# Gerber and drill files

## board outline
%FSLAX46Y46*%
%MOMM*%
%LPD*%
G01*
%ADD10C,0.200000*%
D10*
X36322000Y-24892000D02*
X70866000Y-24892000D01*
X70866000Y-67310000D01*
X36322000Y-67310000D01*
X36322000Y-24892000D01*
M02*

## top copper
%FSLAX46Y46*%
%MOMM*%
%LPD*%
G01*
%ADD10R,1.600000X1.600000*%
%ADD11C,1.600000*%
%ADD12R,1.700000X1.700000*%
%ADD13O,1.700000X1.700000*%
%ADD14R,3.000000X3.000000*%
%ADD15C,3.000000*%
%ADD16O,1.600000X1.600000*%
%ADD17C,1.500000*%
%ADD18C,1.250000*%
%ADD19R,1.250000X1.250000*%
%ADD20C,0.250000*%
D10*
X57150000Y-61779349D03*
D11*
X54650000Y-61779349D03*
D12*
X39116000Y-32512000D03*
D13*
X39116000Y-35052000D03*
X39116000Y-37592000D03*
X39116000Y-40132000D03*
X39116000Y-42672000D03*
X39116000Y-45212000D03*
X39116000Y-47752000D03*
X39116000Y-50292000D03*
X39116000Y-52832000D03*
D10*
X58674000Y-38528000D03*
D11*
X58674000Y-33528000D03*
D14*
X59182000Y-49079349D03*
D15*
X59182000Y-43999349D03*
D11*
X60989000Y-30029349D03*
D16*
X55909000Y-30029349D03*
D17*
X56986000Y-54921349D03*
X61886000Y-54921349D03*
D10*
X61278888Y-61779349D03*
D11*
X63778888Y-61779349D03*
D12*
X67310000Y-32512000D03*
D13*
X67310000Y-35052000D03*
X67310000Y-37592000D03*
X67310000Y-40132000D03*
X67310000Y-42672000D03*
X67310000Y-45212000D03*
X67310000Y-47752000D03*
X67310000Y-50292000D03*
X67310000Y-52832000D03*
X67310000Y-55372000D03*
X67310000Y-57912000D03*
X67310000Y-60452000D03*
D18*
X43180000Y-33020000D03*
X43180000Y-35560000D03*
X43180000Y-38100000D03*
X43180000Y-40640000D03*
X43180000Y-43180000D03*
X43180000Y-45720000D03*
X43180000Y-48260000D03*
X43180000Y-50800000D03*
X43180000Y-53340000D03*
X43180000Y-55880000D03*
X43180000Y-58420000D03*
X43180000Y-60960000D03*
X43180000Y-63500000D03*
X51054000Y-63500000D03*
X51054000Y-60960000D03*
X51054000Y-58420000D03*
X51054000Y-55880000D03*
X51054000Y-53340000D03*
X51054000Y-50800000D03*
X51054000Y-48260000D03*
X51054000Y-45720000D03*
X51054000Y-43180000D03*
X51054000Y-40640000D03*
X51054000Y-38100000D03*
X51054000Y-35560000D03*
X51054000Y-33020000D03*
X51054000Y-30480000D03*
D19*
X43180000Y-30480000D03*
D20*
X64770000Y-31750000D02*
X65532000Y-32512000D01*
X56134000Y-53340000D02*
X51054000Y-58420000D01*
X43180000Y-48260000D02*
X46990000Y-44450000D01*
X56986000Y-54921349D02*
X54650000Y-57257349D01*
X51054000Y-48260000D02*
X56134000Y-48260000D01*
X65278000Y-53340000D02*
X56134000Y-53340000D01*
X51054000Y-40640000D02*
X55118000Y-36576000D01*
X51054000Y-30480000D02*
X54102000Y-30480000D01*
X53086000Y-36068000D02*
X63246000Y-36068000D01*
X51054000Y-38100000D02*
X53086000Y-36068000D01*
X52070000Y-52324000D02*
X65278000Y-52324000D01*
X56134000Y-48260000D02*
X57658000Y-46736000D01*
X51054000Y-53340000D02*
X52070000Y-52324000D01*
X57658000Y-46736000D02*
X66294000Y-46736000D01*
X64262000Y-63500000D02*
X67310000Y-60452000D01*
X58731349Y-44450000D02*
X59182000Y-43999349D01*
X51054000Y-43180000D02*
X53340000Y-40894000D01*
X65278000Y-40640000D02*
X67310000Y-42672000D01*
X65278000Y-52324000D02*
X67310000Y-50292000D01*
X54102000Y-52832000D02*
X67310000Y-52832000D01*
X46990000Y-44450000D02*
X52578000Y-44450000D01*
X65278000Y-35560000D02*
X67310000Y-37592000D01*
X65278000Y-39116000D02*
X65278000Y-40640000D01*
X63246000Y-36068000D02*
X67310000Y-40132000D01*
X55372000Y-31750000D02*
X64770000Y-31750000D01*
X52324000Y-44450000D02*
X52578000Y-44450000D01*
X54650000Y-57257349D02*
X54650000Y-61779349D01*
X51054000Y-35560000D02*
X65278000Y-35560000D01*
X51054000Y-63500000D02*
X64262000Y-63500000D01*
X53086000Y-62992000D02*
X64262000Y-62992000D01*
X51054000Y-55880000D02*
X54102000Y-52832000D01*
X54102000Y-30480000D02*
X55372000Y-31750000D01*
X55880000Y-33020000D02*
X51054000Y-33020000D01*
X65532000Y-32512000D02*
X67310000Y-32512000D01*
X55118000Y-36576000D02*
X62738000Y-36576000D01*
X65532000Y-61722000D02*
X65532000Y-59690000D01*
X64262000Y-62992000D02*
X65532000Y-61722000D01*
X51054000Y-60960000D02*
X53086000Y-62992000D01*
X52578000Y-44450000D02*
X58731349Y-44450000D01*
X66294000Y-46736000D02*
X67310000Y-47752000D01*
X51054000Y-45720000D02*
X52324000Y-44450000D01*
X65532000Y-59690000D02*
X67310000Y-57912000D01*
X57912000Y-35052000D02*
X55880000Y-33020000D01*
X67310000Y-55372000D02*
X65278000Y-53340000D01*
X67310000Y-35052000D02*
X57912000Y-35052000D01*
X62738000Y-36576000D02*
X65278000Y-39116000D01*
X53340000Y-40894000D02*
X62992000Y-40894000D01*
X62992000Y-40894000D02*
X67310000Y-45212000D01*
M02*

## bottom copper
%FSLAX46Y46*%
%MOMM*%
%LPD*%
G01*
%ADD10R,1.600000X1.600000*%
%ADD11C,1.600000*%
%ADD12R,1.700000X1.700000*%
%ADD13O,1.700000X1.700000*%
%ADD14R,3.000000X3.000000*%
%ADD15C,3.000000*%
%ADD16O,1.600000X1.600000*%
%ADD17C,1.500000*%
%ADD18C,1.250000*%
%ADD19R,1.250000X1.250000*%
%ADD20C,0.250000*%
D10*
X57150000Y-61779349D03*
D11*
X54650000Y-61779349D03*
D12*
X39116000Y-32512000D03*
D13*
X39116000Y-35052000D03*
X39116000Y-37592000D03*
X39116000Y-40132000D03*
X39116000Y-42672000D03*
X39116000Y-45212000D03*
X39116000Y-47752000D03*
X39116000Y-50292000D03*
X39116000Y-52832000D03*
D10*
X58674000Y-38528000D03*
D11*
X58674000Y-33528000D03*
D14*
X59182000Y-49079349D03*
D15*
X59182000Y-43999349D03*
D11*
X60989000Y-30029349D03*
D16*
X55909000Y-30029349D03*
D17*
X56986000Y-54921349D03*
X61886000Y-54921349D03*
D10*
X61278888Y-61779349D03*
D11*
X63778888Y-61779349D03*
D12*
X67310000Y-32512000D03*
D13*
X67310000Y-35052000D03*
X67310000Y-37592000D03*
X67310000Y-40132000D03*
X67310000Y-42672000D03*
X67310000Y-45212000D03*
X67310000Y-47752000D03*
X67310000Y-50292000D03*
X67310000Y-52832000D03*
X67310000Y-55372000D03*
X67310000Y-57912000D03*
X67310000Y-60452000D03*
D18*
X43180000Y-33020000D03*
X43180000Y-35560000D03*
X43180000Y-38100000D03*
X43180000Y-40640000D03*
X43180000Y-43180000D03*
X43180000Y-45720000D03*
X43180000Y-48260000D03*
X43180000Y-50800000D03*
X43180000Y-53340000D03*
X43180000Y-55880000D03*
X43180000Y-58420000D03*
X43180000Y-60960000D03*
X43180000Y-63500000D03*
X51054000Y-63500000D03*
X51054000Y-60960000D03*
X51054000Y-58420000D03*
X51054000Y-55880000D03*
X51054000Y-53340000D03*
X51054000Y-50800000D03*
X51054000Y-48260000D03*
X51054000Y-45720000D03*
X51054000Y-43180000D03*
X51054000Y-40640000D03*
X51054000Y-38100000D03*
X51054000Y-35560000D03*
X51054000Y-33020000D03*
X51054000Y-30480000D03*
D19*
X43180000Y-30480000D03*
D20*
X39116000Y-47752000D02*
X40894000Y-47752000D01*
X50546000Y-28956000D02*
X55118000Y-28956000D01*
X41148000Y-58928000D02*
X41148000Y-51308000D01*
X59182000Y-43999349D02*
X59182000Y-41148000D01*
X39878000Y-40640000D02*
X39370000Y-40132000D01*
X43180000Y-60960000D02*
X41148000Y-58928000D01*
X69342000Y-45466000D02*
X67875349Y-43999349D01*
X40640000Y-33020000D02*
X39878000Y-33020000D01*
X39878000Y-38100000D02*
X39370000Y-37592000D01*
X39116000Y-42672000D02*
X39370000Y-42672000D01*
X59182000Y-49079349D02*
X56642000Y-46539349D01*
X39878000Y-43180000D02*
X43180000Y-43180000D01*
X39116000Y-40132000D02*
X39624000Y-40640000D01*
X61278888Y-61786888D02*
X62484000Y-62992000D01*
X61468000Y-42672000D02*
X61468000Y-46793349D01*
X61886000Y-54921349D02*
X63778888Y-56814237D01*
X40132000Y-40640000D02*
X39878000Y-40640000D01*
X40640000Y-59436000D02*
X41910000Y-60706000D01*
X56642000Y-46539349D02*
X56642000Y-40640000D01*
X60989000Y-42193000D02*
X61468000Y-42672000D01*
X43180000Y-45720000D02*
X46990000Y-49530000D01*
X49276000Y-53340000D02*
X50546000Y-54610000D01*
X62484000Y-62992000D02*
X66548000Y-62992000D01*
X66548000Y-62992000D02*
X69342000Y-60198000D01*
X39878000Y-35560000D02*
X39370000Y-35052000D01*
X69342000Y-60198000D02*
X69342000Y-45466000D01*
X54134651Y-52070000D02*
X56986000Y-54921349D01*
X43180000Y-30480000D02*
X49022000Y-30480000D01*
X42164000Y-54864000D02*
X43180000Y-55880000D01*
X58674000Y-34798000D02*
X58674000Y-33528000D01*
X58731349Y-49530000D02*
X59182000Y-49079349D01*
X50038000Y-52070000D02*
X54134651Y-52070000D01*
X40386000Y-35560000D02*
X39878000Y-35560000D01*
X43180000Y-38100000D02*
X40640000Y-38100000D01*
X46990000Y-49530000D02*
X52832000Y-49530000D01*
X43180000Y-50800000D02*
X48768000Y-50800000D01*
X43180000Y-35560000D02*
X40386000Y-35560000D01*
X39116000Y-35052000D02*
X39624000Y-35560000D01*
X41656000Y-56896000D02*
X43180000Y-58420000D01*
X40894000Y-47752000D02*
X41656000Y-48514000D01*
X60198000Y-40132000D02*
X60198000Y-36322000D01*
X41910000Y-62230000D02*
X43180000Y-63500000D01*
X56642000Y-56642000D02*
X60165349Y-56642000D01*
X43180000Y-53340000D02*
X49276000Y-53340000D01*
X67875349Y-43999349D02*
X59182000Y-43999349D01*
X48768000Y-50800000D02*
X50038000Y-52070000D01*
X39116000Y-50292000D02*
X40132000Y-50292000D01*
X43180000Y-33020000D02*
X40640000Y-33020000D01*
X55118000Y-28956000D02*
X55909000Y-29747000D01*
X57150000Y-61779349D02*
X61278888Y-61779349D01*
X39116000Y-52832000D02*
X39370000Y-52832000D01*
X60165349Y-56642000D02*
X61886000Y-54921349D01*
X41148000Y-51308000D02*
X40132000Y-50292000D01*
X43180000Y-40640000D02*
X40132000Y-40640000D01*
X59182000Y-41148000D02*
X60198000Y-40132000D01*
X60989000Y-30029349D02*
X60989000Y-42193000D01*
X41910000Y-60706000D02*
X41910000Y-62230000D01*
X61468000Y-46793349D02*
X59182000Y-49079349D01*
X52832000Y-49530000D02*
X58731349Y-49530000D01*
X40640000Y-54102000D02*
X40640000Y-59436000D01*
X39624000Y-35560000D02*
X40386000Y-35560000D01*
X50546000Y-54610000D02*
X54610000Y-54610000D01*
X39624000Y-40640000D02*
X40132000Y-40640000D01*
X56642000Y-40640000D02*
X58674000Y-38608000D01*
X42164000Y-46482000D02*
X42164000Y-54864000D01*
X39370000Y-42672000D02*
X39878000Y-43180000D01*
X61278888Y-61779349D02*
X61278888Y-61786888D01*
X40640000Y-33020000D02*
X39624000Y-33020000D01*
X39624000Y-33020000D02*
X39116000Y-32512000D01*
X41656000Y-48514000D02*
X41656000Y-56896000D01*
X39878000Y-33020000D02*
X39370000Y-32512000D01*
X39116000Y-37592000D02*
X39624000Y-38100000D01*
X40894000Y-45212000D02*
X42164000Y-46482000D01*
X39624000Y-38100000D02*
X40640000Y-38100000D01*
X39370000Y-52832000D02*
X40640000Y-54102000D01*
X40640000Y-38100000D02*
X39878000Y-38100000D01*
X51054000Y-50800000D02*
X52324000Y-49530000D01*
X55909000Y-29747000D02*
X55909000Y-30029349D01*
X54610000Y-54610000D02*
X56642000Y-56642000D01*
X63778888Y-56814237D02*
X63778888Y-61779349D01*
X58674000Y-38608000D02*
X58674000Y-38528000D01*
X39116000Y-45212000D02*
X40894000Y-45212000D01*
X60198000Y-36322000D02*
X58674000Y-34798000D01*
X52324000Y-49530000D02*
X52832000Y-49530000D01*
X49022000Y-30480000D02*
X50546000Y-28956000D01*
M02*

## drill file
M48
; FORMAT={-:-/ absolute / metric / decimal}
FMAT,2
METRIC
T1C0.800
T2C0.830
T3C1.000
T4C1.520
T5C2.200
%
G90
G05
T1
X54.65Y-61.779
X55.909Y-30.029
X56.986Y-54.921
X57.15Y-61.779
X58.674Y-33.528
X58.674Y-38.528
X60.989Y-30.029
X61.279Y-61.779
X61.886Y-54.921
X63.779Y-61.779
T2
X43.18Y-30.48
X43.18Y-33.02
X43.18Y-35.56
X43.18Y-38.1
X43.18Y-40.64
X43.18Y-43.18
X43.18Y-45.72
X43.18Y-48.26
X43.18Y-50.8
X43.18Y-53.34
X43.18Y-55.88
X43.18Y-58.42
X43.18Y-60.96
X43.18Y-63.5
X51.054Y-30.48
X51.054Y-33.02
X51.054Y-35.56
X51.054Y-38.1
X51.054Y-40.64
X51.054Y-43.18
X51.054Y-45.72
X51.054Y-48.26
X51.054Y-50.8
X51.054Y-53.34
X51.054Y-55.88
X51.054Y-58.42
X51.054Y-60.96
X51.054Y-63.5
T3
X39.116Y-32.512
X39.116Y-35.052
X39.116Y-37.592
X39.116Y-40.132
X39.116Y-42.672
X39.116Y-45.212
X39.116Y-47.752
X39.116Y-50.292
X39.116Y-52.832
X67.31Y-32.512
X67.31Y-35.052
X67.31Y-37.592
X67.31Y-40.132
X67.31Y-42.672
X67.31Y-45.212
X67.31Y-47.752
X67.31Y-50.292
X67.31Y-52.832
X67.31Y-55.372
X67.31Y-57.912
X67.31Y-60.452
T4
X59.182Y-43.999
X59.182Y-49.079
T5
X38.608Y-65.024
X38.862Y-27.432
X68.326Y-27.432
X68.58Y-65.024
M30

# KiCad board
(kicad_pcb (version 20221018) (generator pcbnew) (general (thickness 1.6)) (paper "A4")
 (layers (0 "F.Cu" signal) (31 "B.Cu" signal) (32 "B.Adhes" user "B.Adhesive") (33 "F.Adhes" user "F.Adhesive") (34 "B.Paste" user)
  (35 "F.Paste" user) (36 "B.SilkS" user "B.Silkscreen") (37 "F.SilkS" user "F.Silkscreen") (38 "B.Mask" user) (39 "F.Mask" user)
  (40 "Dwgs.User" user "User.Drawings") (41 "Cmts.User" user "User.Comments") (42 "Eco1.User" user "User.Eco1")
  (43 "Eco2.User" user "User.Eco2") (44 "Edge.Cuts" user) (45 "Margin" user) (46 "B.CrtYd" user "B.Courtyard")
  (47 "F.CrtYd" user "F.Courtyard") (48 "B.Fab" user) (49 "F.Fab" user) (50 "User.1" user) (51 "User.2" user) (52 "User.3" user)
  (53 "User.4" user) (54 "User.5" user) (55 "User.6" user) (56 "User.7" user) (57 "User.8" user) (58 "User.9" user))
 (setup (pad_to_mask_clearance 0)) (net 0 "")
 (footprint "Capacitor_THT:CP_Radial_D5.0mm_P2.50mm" (layer "F.Cu") (at 57.15 61.779349 180)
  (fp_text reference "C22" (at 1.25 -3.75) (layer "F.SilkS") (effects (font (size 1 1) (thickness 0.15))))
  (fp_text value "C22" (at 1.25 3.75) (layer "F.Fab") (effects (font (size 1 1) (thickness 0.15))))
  (pad "1" thru_hole rect (at 0 0 180) (size 1.6 1.6) (drill 0.8) (layers "*.Cu" "*.Mask"))
  (pad "2" thru_hole circle (at 2.5 0 180) (size 1.6 1.6) (drill 0.8) (layers "*.Cu" "*.Mask")))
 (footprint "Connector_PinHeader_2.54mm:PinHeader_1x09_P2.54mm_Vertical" (layer "F.Cu") (at 39.116 32.512)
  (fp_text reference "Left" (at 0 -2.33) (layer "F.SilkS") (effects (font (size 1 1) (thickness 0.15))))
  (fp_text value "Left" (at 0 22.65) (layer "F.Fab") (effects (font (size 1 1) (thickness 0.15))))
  (pad "1" thru_hole rect (at 0 0) (size 1.7 1.7) (drill 1) (layers "*.Cu" "*.Mask"))
  (pad "2" thru_hole oval (at 0 2.54) (size 1.7 1.7) (drill 1) (layers "*.Cu" "*.Mask"))
  (pad "3" thru_hole oval (at 0 5.08) (size 1.7 1.7) (drill 1) (layers "*.Cu" "*.Mask"))
  (pad "4" thru_hole oval (at 0 7.62) (size 1.7 1.7) (drill 1) (layers "*.Cu" "*.Mask"))
  (pad "5" thru_hole oval (at 0 10.16) (size 1.7 1.7) (drill 1) (layers "*.Cu" "*.Mask"))
  (pad "6" thru_hole oval (at 0 12.7) (size 1.7 1.7) (drill 1) (layers "*.Cu" "*.Mask"))
  (pad "7" thru_hole oval (at 0 15.24) (size 1.7 1.7) (drill 1) (layers "*.Cu" "*.Mask"))
  (pad "8" thru_hole oval (at 0 17.78) (size 1.7 1.7) (drill 1) (layers "*.Cu" "*.Mask"))
  (pad "9" thru_hole oval (at 0 20.32) (size 1.7 1.7) (drill 1) (layers "*.Cu" "*.Mask")))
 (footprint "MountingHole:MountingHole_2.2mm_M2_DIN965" (layer "F.Cu") (at 38.608 65.024)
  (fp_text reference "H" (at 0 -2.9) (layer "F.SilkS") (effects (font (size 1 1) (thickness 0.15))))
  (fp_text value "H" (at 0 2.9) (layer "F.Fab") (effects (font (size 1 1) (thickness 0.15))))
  (pad "" np_thru_hole circle (at 0 0) (size 2.2 2.2) (drill 2.2) (layers "*.Cu" "*.Mask")))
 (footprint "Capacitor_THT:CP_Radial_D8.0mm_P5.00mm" (layer "F.Cu") (at 58.674 38.528 90)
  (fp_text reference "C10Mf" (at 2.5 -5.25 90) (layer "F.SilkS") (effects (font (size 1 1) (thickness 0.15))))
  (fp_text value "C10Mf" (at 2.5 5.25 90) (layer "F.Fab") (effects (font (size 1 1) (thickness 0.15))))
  (pad "+" thru_hole rect (at 0 0 90) (size 1.6 1.6) (drill 0.8) (layers "*.Cu" "*.Mask"))
  (pad "-" thru_hole circle (at 5 0 90) (size 1.6 1.6) (drill 0.8) (layers "*.Cu" "*.Mask")))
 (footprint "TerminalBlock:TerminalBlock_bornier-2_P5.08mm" (layer "F.Cu") (at 59.182 49.079349 90)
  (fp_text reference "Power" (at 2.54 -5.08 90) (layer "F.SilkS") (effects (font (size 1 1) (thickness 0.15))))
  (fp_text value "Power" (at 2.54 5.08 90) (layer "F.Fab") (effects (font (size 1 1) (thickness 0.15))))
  (pad "+5v" thru_hole rect (at 0 0 90) (size 3 3) (drill 1.52) (layers "*.Cu" "*.Mask"))
  (pad "GND" thru_hole circle (at 5.08 0 90) (size 3 3) (drill 1.52) (layers "*.Cu" "*.Mask")))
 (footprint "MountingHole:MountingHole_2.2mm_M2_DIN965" (layer "F.Cu") (at 68.58 65.024)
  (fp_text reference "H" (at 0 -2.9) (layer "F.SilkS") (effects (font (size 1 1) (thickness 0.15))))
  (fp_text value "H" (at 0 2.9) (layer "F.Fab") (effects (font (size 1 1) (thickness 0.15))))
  (pad "" np_thru_hole circle (at 0 0) (size 2.2 2.2) (drill 2.2) (layers "*.Cu" "*.Mask")))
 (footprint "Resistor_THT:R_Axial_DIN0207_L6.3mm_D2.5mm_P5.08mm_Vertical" (layer "F.Cu") (at 60.989 30.029349 180)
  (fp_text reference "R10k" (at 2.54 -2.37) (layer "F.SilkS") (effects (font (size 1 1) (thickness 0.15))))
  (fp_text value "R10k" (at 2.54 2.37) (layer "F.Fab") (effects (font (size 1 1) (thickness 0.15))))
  (pad "1" thru_hole circle (at 0 0 180) (size 1.6 1.6) (drill 0.8) (layers "*.Cu" "*.Mask"))
  (pad "2" thru_hole oval (at 5.08 0 180) (size 1.6 1.6) (drill 0.8) (layers "*.Cu" "*.Mask")))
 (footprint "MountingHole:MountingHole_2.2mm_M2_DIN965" (layer "F.Cu") (at 38.862 27.432)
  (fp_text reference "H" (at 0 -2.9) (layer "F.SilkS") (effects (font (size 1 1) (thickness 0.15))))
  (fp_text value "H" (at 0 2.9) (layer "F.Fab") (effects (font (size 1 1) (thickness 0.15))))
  (pad "" np_thru_hole circle (at 0 0) (size 2.2 2.2) (drill 2.2) (layers "F&B.Cu" "*.Mask")))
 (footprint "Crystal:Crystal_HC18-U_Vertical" (layer "F.Cu") (at 56.986 54.921349)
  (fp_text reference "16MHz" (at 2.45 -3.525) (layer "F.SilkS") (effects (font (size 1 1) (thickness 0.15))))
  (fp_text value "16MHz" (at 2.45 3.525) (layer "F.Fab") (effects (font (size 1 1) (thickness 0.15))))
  (pad "1" thru_hole circle (at 0 0) (size 1.5 1.5) (drill 0.8) (layers "*.Cu" "*.Mask"))
  (pad "2" thru_hole circle (at 4.9 0) (size 1.5 1.5) (drill 0.8) (layers "*.Cu" "*.Mask")))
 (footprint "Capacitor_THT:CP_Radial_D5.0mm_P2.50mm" (layer "F.Cu") (at 61.278888 61.779349)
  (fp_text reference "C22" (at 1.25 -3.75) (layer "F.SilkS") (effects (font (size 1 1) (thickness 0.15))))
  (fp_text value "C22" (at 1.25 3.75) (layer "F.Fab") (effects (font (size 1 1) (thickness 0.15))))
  (pad "1" thru_hole rect (at 0 0) (size 1.6 1.6) (drill 0.8) (layers "*.Cu" "*.Mask"))
  (pad "2" thru_hole circle (at 2.5 0) (size 1.6 1.6) (drill 0.8) (layers "*.Cu" "*.Mask")))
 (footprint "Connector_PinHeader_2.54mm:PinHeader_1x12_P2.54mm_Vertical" (layer "F.Cu") (at 67.31 32.512)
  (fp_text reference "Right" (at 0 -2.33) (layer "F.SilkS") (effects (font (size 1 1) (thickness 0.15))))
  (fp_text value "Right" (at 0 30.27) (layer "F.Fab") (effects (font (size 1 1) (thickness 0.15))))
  (pad "1" thru_hole rect (at 0 0) (size 1.7 1.7) (drill 1) (layers "*.Cu" "*.Mask"))
  (pad "2" thru_hole oval (at 0 2.54) (size 1.7 1.7) (drill 1) (layers "*.Cu" "*.Mask"))
  (pad "3" thru_hole oval (at 0 5.08) (size 1.7 1.7) (drill 1) (layers "*.Cu" "*.Mask"))
  (pad "4" thru_hole oval (at 0 7.62) (size 1.7 1.7) (drill 1) (layers "*.Cu" "*.Mask"))
  (pad "5" thru_hole oval (at 0 10.16) (size 1.7 1.7) (drill 1) (layers "*.Cu" "*.Mask"))
  (pad "6" thru_hole oval (at 0 12.7) (size 1.7 1.7) (drill 1) (layers "*.Cu" "*.Mask"))
  (pad "7" thru_hole oval (at 0 15.24) (size 1.7 1.7) (drill 1) (layers "*.Cu" "*.Mask"))
  (pad "8" thru_hole oval (at 0 17.78) (size 1.7 1.7) (drill 1) (layers "*.Cu" "*.Mask"))
  (pad "9" thru_hole oval (at 0 20.32) (size 1.7 1.7) (drill 1) (layers "*.Cu" "*.Mask"))
  (pad "10" thru_hole oval (at 0 22.86) (size 1.7 1.7) (drill 1) (layers "*.Cu" "*.Mask"))
  (pad "11" thru_hole oval (at 0 25.4) (size 1.7 1.7) (drill 1) (layers "*.Cu" "*.Mask"))
  (pad "12" thru_hole oval (at 0 27.94) (size 1.7 1.7) (drill 1) (layers "*.Cu" "*.Mask")))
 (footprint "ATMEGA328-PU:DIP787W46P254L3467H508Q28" (layer "F.Cu") (at 47.117 46.99)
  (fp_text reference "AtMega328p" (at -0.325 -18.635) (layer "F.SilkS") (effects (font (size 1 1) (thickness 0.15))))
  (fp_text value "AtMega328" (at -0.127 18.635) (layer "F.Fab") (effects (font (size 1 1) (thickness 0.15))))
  (pad "2" thru_hole circle (at -3.937 -13.97) (size 1.25 1.25) (drill 0.83) (layers "*.Cu" "*.Mask") (solder_mask_margin 0.102))
  (pad "3" thru_hole circle (at -3.937 -11.43) (size 1.25 1.25) (drill 0.83) (layers "*.Cu" "*.Mask") (solder_mask_margin 0.102))
  (pad "4" thru_hole circle (at -3.937 -8.89) (size 1.25 1.25) (drill 0.83) (layers "*.Cu" "*.Mask") (solder_mask_margin 0.102))
  (pad "5" thru_hole circle (at -3.937 -6.35) (size 1.25 1.25) (drill 0.83) (layers "*.Cu" "*.Mask") (solder_mask_margin 0.102))
  (pad "6" thru_hole circle (at -3.937 -3.81) (size 1.25 1.25) (drill 0.83) (layers "*.Cu" "*.Mask") (solder_mask_margin 0.102))
  (pad "7" thru_hole circle (at -3.937 -1.27) (size 1.25 1.25) (drill 0.83) (layers "*.Cu" "*.Mask") (solder_mask_margin 0.102))
  (pad "8" thru_hole circle (at -3.937 1.27) (size 1.25 1.25) (drill 0.83) (layers "*.Cu" "*.Mask") (solder_mask_margin 0.102))
  (pad "9" thru_hole circle (at -3.937 3.81) (size 1.25 1.25) (drill 0.83) (layers "*.Cu" "*.Mask") (solder_mask_margin 0.102))
  (pad "10" thru_hole circle (at -3.937 6.35) (size 1.25 1.25) (drill 0.83) (layers "*.Cu" "*.Mask") (solder_mask_margin 0.102))
  (pad "11" thru_hole circle (at -3.937 8.89) (size 1.25 1.25) (drill 0.83) (layers "*.Cu" "*.Mask") (solder_mask_margin 0.102))
  (pad "12" thru_hole circle (at -3.937 11.43) (size 1.25 1.25) (drill 0.83) (layers "*.Cu" "*.Mask") (solder_mask_margin 0.102))
  (pad "13" thru_hole circle (at -3.937 13.97) (size 1.25 1.25) (drill 0.83) (layers "*.Cu" "*.Mask") (solder_mask_margin 0.102))
  (pad "14" thru_hole circle (at -3.937 16.51) (size 1.25 1.25) (drill 0.83) (layers "*.Cu" "*.Mask") (solder_mask_margin 0.102))
  (pad "15" thru_hole circle (at 3.937 16.51) (size 1.25 1.25) (drill 0.83) (layers "*.Cu" "*.Mask") (solder_mask_margin 0.102))
  (pad "16" thru_hole circle (at 3.937 13.97) (size 1.25 1.25) (drill 0.83) (layers "*.Cu" "*.Mask") (solder_mask_margin 0.102))
  (pad "17" thru_hole circle (at 3.937 11.43) (size 1.25 1.25) (drill 0.83) (layers "*.Cu" "*.Mask") (solder_mask_margin 0.102))
  (pad "18" thru_hole circle (at 3.937 8.89) (size 1.25 1.25) (drill 0.83) (layers "*.Cu" "*.Mask") (solder_mask_margin 0.102))
  (pad "19" thru_hole circle (at 3.937 6.35) (size 1.25 1.25) (drill 0.83) (layers "*.Cu" "*.Mask") (solder_mask_margin 0.102))
  (pad "20" thru_hole circle (at 3.937 3.81) (size 1.25 1.25) (drill 0.83) (layers "*.Cu" "*.Mask") (solder_mask_margin 0.102))
  (pad "21" thru_hole circle (at 3.937 1.27) (size 1.25 1.25) (drill 0.83) (layers "*.Cu" "*.Mask") (solder_mask_margin 0.102))
  (pad "22" thru_hole circle (at 3.937 -1.27) (size 1.25 1.25) (drill 0.83) (layers "*.Cu" "*.Mask") (solder_mask_margin 0.102))
  (pad "23" thru_hole circle (at 3.937 -3.81) (size 1.25 1.25) (drill 0.83) (layers "*.Cu" "*.Mask") (solder_mask_margin 0.102))
  (pad "24" thru_hole circle (at 3.937 -6.35) (size 1.25 1.25) (drill 0.83) (layers "*.Cu" "*.Mask") (solder_mask_margin 0.102))
  (pad "25" thru_hole circle (at 3.937 -8.89) (size 1.25 1.25) (drill 0.83) (layers "*.Cu" "*.Mask") (solder_mask_margin 0.102))
  (pad "26" thru_hole circle (at 3.937 -11.43) (size 1.25 1.25) (drill 0.83) (layers "*.Cu" "*.Mask") (solder_mask_margin 0.102))
  (pad "27" thru_hole circle (at 3.937 -13.97) (size 1.25 1.25) (drill 0.83) (layers "*.Cu" "*.Mask") (solder_mask_margin 0.102))
  (pad "28" thru_hole circle (at 3.937 -16.51) (size 1.25 1.25) (drill 0.83) (layers "*.Cu" "*.Mask") (solder_mask_margin 0.102))
  (pad "RESET" thru_hole rect (at -3.937 -16.51) (size 1.25 1.25) (drill 0.83) (layers "*.Cu" "*.Mask") (solder_mask_margin 0.102)))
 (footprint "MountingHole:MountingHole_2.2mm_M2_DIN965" (layer "F.Cu") (at 68.326 27.432)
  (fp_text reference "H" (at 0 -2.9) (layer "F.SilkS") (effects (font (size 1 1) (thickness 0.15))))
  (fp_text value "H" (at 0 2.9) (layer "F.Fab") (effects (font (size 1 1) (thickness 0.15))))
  (pad "" np_thru_hole circle (at 0 0) (size 2.2 2.2) (drill 2.2) (layers "*.Cu" "*.Mask")))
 (gr_rect (start 36.322 24.892) (end 70.866 67.31) (stroke (width 0.2) (type default)) (fill none) (layer "Edge.Cuts"))
 (segment (start 64.77 31.75) (end 65.532 32.512) (width 0.25) (layer "F.Cu") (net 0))
 (segment (start 56.134 53.34) (end 51.054 58.42) (width 0.25) (layer "F.Cu") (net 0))
 (segment (start 43.18 48.26) (end 46.99 44.45) (width 0.25) (layer "F.Cu") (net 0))
 (segment (start 56.986 54.921349) (end 54.65 57.257349) (width 0.25) (layer "F.Cu") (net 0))
 (segment (start 51.054 48.26) (end 56.134 48.26) (width 0.25) (layer "F.Cu") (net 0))
 (segment (start 65.278 53.34) (end 56.134 53.34) (width 0.25) (layer "F.Cu") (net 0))
 (segment (start 51.054 40.64) (end 55.118 36.576) (width 0.25) (layer "F.Cu") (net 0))
 (segment (start 51.054 30.48) (end 54.102 30.48) (width 0.25) (layer "F.Cu") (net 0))
 (segment (start 53.086 36.068) (end 63.246 36.068) (width 0.25) (layer "F.Cu") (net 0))
 (segment (start 51.054 38.1) (end 53.086 36.068) (width 0.25) (layer "F.Cu") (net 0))
 (segment (start 52.07 52.324) (end 65.278 52.324) (width 0.25) (layer "F.Cu") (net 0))
 (segment (start 56.134 48.26) (end 57.658 46.736) (width 0.25) (layer "F.Cu") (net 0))
 (segment (start 51.054 53.34) (end 52.07 52.324) (width 0.25) (layer "F.Cu") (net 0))
 (segment (start 57.658 46.736) (end 66.294 46.736) (width 0.25) (layer "F.Cu") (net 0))
 (segment (start 64.262 63.5) (end 67.31 60.452) (width 0.25) (layer "F.Cu") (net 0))
 (segment (start 58.731349 44.45) (end 59.182 43.999349) (width 0.25) (layer "F.Cu") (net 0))
 (segment (start 51.054 43.18) (end 53.34 40.894) (width 0.25) (layer "F.Cu") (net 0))
 (segment (start 65.278 40.64) (end 67.31 42.672) (width 0.25) (layer "F.Cu") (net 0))
 (segment (start 65.278 52.324) (end 67.31 50.292) (width 0.25) (layer "F.Cu") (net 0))
 (segment (start 54.102 52.832) (end 67.31 52.832) (width 0.25) (layer "F.Cu") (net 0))
 (segment (start 46.99 44.45) (end 52.578 44.45) (width 0.25) (layer "F.Cu") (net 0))
 (segment (start 65.278 35.56) (end 67.31 37.592) (width 0.25) (layer "F.Cu") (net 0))
 (segment (start 65.278 39.116) (end 65.278 40.64) (width 0.25) (layer "F.Cu") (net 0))
 (segment (start 63.246 36.068) (end 67.31 40.132) (width 0.25) (layer "F.Cu") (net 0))
 (segment (start 55.372 31.75) (end 64.77 31.75) (width 0.25) (layer "F.Cu") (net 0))
 (segment (start 52.324 44.45) (end 52.578 44.45) (width 0.25) (layer "F.Cu") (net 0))
 (segment (start 54.65 57.257349) (end 54.65 61.779349) (width 0.25) (layer "F.Cu") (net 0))
 (segment (start 51.054 35.56) (end 65.278 35.56) (width 0.25) (layer "F.Cu") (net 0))
 (segment (start 51.054 63.5) (end 64.262 63.5) (width 0.25) (layer "F.Cu") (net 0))
 (segment (start 53.086 62.992) (end 64.262 62.992) (width 0.25) (layer "F.Cu") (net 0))
 (segment (start 51.054 55.88) (end 54.102 52.832) (width 0.25) (layer "F.Cu") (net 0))
 (segment (start 54.102 30.48) (end 55.372 31.75) (width 0.25) (layer "F.Cu") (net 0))
 (segment (start 55.88 33.02) (end 51.054 33.02) (width 0.25) (layer "F.Cu") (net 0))
 (segment (start 65.532 32.512) (end 67.31 32.512) (width 0.25) (layer "F.Cu") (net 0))
 (segment (start 55.118 36.576) (end 62.738 36.576) (width 0.25) (layer "F.Cu") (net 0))
 (segment (start 65.532 61.722) (end 65.532 59.69) (width 0.25) (layer "F.Cu") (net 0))
 (segment (start 64.262 62.992) (end 65.532 61.722) (width 0.25) (layer "F.Cu") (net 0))
 (segment (start 51.054 60.96) (end 53.086 62.992) (width 0.25) (layer "F.Cu") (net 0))
 (segment (start 52.578 44.45) (end 58.731349 44.45) (width 0.25) (layer "F.Cu") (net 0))
 (segment (start 66.294 46.736) (end 67.31 47.752) (width 0.25) (layer "F.Cu") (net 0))
 (segment (start 51.054 45.72) (end 52.324 44.45) (width 0.25) (layer "F.Cu") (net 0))
 (segment (start 65.532 59.69) (end 67.31 57.912) (width 0.25) (layer "F.Cu") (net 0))
 (segment (start 57.912 35.052) (end 55.88 33.02) (width 0.25) (layer "F.Cu") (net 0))
 (segment (start 67.31 55.372) (end 65.278 53.34) (width 0.25) (layer "F.Cu") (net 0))
 (segment (start 67.31 35.052) (end 57.912 35.052) (width 0.25) (layer "F.Cu") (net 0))
 (segment (start 62.738 36.576) (end 65.278 39.116) (width 0.25) (layer "F.Cu") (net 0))
 (segment (start 53.34 40.894) (end 62.992 40.894) (width 0.25) (layer "F.Cu") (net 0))
 (segment (start 62.992 40.894) (end 67.31 45.212) (width 0.25) (layer "F.Cu") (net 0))
 (segment (start 39.116 47.752) (end 40.894 47.752) (width 0.25) (layer "B.Cu") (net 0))
 (segment (start 50.546 28.956) (end 55.118 28.956) (width 0.25) (layer "B.Cu") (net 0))
 (segment (start 41.148 58.928) (end 41.148 51.308) (width 0.25) (layer "B.Cu") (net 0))
 (segment (start 59.182 43.999349) (end 59.182 41.148) (width 0.25) (layer "B.Cu") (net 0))
 (segment (start 39.878 40.64) (end 39.37 40.132) (width 0.25) (layer "B.Cu") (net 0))
 (segment (start 43.18 60.96) (end 41.148 58.928) (width 0.25) (layer "B.Cu") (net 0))
 (segment (start 69.342 45.466) (end 67.875349 43.999349) (width 0.25) (layer "B.Cu") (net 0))
 (segment (start 40.64 33.02) (end 39.878 33.02) (width 0.25) (layer "B.Cu") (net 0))
 (segment (start 39.878 38.1) (end 39.37 37.592) (width 0.25) (layer "B.Cu") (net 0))
 (segment (start 39.116 42.672) (end 39.37 42.672) (width 0.25) (layer "B.Cu") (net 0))
 (segment (start 59.182 49.079349) (end 56.642 46.539349) (width 0.25) (layer "B.Cu") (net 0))
 (segment (start 39.878 43.18) (end 43.18 43.18) (width 0.25) (layer "B.Cu") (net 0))
 (segment (start 39.116 40.132) (end 39.624 40.64) (width 0.25) (layer "B.Cu") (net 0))
 (segment (start 61.278888 61.786888) (end 62.484 62.992) (width 0.25) (layer "B.Cu") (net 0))
 (segment (start 61.468 42.672) (end 61.468 46.793349) (width 0.25) (layer "B.Cu") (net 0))
 (segment (start 61.886 54.921349) (end 63.778888 56.814237) (width 0.25) (layer "B.Cu") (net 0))
 (segment (start 40.132 40.64) (end 39.878 40.64) (width 0.25) (layer "B.Cu") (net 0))
 (segment (start 40.64 59.436) (end 41.91 60.706) (width 0.25) (layer "B.Cu") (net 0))
 (segment (start 56.642 46.539349) (end 56.642 40.64) (width 0.25) (layer "B.Cu") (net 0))
 (segment (start 60.989 42.193) (end 61.468 42.672) (width 0.25) (layer "B.Cu") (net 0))
 (segment (start 43.18 45.72) (end 46.99 49.53) (width 0.25) (layer "B.Cu") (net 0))
 (segment (start 49.276 53.34) (end 50.546 54.61) (width 0.25) (layer "B.Cu") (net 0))
 (segment (start 62.484 62.992) (end 66.548 62.992) (width 0.25) (layer "B.Cu") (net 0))
 (segment (start 66.548 62.992) (end 69.342 60.198) (width 0.25) (layer "B.Cu") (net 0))
 (segment (start 39.878 35.56) (end 39.37 35.052) (width 0.25) (layer "B.Cu") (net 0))
 (segment (start 69.342 60.198) (end 69.342 45.466) (width 0.25) (layer "B.Cu") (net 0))
 (segment (start 54.134651 52.07) (end 56.986 54.921349) (width 0.25) (layer "B.Cu") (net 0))
 (segment (start 43.18 30.48) (end 49.022 30.48) (width 0.25) (layer "B.Cu") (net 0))
 (segment (start 42.164 54.864) (end 43.18 55.88) (width 0.25) (layer "B.Cu") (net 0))
 (segment (start 58.674 34.798) (end 58.674 33.528) (width 0.25) (layer "B.Cu") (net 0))
 (segment (start 58.731349 49.53) (end 59.182 49.079349) (width 0.25) (layer "B.Cu") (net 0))
 (segment (start 50.038 52.07) (end 54.134651 52.07) (width 0.25) (layer "B.Cu") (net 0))
 (segment (start 40.386 35.56) (end 39.878 35.56) (width 0.25) (layer "B.Cu") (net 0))
 (segment (start 43.18 38.1) (end 40.64 38.1) (width 0.25) (layer "B.Cu") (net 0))
 (segment (start 46.99 49.53) (end 52.832 49.53) (width 0.25) (layer "B.Cu") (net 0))
 (segment (start 43.18 50.8) (end 48.768 50.8) (width 0.25) (layer "B.Cu") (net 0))
 (segment (start 43.18 35.56) (end 40.386 35.56) (width 0.25) (layer "B.Cu") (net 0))
 (segment (start 39.116 35.052) (end 39.624 35.56) (width 0.25) (layer "B.Cu") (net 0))
 (segment (start 41.656 56.896) (end 43.18 58.42) (width 0.25) (layer "B.Cu") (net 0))
 (segment (start 40.894 47.752) (end 41.656 48.514) (width 0.25) (layer "B.Cu") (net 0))
 (segment (start 60.198 40.132) (end 60.198 36.322) (width 0.25) (layer "B.Cu") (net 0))
 (segment (start 41.91 62.23) (end 43.18 63.5) (width 0.25) (layer "B.Cu") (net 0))
 (segment (start 56.642 56.642) (end 60.165349 56.642) (width 0.25) (layer "B.Cu") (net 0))
 (segment (start 43.18 53.34) (end 49.276 53.34) (width 0.25) (layer "B.Cu") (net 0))
 (segment (start 67.875349 43.999349) (end 59.182 43.999349) (width 0.25) (layer "B.Cu") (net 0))
 (segment (start 48.768 50.8) (end 50.038 52.07) (width 0.25) (layer "B.Cu") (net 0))
 (segment (start 39.116 50.292) (end 40.132 50.292) (width 0.25) (layer "B.Cu") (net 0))
 (segment (start 43.18 33.02) (end 40.64 33.02) (width 0.25) (layer "B.Cu") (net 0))
 (segment (start 55.118 28.956) (end 55.909 29.747) (width 0.25) (layer "B.Cu") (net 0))
 (segment (start 57.15 61.779349) (end 61.278888 61.779349) (width 0.25) (layer "B.Cu") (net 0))
 (segment (start 39.116 52.832) (end 39.37 52.832) (width 0.25) (layer "B.Cu") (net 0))
 (segment (start 60.165349 56.642) (end 61.886 54.921349) (width 0.25) (layer "B.Cu") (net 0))
 (segment (start 41.148 51.308) (end 40.132 50.292) (width 0.25) (layer "B.Cu") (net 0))
 (segment (start 43.18 40.64) (end 40.132 40.64) (width 0.25) (layer "B.Cu") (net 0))
 (segment (start 59.182 41.148) (end 60.198 40.132) (width 0.25) (layer "B.Cu") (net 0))
 (segment (start 60.989 30.029349) (end 60.989 42.193) (width 0.25) (layer "B.Cu") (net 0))
 (segment (start 41.91 60.706) (end 41.91 62.23) (width 0.25) (layer "B.Cu") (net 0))
 (segment (start 61.468 46.793349) (end 59.182 49.079349) (width 0.25) (layer "B.Cu") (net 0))
 (segment (start 52.832 49.53) (end 58.731349 49.53) (width 0.25) (layer "B.Cu") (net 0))
 (segment (start 40.64 54.102) (end 40.64 59.436) (width 0.25) (layer "B.Cu") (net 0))
 (segment (start 39.624 35.56) (end 40.386 35.56) (width 0.25) (layer "B.Cu") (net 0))
 (segment (start 50.546 54.61) (end 54.61 54.61) (width 0.25) (layer "B.Cu") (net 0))
 (segment (start 39.624 40.64) (end 40.132 40.64) (width 0.25) (layer "B.Cu") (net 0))
 (segment (start 56.642 40.64) (end 58.674 38.608) (width 0.25) (layer "B.Cu") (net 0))
 (segment (start 42.164 46.482) (end 42.164 54.864) (width 0.25) (layer "B.Cu") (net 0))
 (segment (start 39.37 42.672) (end 39.878 43.18) (width 0.25) (layer "B.Cu") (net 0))
 (segment (start 61.278888 61.779349) (end 61.278888 61.786888) (width 0.25) (layer "B.Cu") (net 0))
 (segment (start 40.64 33.02) (end 39.624 33.02) (width 0.25) (layer "B.Cu") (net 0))
 (segment (start 39.624 33.02) (end 39.116 32.512) (width 0.25) (layer "B.Cu") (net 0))
 (segment (start 41.656 48.514) (end 41.656 56.896) (width 0.25) (layer "B.Cu") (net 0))
 (segment (start 39.878 33.02) (end 39.37 32.512) (width 0.25) (layer "B.Cu") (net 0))
 (segment (start 39.116 37.592) (end 39.624 38.1) (width 0.25) (layer "B.Cu") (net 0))
 (segment (start 40.894 45.212) (end 42.164 46.482) (width 0.25) (layer "B.Cu") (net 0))
 (segment (start 39.624 38.1) (end 40.64 38.1) (width 0.25) (layer "B.Cu") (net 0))
 (segment (start 39.37 52.832) (end 40.64 54.102) (width 0.25) (layer "B.Cu") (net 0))
 (segment (start 40.64 38.1) (end 39.878 38.1) (width 0.25) (layer "B.Cu") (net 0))
 (segment (start 51.054 50.8) (end 52.324 49.53) (width 0.25) (layer "B.Cu") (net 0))
 (segment (start 55.909 29.747) (end 55.909 30.029349) (width 0.25) (layer "B.Cu") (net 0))
 (segment (start 54.61 54.61) (end 56.642 56.642) (width 0.25) (layer "B.Cu") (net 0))
 (segment (start 63.778888 56.814237) (end 63.778888 61.779349) (width 0.25) (layer "B.Cu") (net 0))
 (segment (start 58.674 38.608) (end 58.674 38.528) (width 0.25) (layer "B.Cu") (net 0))
 (segment (start 39.116 45.212) (end 40.894 45.212) (width 0.25) (layer "B.Cu") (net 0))
 (segment (start 60.198 36.322) (end 58.674 34.798) (width 0.25) (layer "B.Cu") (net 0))
 (segment (start 52.324 49.53) (end 52.832 49.53) (width 0.25) (layer "B.Cu") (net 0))
 (segment (start 49.022 30.48) (end 50.546 28.956) (width 0.25) (layer "B.Cu") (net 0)))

